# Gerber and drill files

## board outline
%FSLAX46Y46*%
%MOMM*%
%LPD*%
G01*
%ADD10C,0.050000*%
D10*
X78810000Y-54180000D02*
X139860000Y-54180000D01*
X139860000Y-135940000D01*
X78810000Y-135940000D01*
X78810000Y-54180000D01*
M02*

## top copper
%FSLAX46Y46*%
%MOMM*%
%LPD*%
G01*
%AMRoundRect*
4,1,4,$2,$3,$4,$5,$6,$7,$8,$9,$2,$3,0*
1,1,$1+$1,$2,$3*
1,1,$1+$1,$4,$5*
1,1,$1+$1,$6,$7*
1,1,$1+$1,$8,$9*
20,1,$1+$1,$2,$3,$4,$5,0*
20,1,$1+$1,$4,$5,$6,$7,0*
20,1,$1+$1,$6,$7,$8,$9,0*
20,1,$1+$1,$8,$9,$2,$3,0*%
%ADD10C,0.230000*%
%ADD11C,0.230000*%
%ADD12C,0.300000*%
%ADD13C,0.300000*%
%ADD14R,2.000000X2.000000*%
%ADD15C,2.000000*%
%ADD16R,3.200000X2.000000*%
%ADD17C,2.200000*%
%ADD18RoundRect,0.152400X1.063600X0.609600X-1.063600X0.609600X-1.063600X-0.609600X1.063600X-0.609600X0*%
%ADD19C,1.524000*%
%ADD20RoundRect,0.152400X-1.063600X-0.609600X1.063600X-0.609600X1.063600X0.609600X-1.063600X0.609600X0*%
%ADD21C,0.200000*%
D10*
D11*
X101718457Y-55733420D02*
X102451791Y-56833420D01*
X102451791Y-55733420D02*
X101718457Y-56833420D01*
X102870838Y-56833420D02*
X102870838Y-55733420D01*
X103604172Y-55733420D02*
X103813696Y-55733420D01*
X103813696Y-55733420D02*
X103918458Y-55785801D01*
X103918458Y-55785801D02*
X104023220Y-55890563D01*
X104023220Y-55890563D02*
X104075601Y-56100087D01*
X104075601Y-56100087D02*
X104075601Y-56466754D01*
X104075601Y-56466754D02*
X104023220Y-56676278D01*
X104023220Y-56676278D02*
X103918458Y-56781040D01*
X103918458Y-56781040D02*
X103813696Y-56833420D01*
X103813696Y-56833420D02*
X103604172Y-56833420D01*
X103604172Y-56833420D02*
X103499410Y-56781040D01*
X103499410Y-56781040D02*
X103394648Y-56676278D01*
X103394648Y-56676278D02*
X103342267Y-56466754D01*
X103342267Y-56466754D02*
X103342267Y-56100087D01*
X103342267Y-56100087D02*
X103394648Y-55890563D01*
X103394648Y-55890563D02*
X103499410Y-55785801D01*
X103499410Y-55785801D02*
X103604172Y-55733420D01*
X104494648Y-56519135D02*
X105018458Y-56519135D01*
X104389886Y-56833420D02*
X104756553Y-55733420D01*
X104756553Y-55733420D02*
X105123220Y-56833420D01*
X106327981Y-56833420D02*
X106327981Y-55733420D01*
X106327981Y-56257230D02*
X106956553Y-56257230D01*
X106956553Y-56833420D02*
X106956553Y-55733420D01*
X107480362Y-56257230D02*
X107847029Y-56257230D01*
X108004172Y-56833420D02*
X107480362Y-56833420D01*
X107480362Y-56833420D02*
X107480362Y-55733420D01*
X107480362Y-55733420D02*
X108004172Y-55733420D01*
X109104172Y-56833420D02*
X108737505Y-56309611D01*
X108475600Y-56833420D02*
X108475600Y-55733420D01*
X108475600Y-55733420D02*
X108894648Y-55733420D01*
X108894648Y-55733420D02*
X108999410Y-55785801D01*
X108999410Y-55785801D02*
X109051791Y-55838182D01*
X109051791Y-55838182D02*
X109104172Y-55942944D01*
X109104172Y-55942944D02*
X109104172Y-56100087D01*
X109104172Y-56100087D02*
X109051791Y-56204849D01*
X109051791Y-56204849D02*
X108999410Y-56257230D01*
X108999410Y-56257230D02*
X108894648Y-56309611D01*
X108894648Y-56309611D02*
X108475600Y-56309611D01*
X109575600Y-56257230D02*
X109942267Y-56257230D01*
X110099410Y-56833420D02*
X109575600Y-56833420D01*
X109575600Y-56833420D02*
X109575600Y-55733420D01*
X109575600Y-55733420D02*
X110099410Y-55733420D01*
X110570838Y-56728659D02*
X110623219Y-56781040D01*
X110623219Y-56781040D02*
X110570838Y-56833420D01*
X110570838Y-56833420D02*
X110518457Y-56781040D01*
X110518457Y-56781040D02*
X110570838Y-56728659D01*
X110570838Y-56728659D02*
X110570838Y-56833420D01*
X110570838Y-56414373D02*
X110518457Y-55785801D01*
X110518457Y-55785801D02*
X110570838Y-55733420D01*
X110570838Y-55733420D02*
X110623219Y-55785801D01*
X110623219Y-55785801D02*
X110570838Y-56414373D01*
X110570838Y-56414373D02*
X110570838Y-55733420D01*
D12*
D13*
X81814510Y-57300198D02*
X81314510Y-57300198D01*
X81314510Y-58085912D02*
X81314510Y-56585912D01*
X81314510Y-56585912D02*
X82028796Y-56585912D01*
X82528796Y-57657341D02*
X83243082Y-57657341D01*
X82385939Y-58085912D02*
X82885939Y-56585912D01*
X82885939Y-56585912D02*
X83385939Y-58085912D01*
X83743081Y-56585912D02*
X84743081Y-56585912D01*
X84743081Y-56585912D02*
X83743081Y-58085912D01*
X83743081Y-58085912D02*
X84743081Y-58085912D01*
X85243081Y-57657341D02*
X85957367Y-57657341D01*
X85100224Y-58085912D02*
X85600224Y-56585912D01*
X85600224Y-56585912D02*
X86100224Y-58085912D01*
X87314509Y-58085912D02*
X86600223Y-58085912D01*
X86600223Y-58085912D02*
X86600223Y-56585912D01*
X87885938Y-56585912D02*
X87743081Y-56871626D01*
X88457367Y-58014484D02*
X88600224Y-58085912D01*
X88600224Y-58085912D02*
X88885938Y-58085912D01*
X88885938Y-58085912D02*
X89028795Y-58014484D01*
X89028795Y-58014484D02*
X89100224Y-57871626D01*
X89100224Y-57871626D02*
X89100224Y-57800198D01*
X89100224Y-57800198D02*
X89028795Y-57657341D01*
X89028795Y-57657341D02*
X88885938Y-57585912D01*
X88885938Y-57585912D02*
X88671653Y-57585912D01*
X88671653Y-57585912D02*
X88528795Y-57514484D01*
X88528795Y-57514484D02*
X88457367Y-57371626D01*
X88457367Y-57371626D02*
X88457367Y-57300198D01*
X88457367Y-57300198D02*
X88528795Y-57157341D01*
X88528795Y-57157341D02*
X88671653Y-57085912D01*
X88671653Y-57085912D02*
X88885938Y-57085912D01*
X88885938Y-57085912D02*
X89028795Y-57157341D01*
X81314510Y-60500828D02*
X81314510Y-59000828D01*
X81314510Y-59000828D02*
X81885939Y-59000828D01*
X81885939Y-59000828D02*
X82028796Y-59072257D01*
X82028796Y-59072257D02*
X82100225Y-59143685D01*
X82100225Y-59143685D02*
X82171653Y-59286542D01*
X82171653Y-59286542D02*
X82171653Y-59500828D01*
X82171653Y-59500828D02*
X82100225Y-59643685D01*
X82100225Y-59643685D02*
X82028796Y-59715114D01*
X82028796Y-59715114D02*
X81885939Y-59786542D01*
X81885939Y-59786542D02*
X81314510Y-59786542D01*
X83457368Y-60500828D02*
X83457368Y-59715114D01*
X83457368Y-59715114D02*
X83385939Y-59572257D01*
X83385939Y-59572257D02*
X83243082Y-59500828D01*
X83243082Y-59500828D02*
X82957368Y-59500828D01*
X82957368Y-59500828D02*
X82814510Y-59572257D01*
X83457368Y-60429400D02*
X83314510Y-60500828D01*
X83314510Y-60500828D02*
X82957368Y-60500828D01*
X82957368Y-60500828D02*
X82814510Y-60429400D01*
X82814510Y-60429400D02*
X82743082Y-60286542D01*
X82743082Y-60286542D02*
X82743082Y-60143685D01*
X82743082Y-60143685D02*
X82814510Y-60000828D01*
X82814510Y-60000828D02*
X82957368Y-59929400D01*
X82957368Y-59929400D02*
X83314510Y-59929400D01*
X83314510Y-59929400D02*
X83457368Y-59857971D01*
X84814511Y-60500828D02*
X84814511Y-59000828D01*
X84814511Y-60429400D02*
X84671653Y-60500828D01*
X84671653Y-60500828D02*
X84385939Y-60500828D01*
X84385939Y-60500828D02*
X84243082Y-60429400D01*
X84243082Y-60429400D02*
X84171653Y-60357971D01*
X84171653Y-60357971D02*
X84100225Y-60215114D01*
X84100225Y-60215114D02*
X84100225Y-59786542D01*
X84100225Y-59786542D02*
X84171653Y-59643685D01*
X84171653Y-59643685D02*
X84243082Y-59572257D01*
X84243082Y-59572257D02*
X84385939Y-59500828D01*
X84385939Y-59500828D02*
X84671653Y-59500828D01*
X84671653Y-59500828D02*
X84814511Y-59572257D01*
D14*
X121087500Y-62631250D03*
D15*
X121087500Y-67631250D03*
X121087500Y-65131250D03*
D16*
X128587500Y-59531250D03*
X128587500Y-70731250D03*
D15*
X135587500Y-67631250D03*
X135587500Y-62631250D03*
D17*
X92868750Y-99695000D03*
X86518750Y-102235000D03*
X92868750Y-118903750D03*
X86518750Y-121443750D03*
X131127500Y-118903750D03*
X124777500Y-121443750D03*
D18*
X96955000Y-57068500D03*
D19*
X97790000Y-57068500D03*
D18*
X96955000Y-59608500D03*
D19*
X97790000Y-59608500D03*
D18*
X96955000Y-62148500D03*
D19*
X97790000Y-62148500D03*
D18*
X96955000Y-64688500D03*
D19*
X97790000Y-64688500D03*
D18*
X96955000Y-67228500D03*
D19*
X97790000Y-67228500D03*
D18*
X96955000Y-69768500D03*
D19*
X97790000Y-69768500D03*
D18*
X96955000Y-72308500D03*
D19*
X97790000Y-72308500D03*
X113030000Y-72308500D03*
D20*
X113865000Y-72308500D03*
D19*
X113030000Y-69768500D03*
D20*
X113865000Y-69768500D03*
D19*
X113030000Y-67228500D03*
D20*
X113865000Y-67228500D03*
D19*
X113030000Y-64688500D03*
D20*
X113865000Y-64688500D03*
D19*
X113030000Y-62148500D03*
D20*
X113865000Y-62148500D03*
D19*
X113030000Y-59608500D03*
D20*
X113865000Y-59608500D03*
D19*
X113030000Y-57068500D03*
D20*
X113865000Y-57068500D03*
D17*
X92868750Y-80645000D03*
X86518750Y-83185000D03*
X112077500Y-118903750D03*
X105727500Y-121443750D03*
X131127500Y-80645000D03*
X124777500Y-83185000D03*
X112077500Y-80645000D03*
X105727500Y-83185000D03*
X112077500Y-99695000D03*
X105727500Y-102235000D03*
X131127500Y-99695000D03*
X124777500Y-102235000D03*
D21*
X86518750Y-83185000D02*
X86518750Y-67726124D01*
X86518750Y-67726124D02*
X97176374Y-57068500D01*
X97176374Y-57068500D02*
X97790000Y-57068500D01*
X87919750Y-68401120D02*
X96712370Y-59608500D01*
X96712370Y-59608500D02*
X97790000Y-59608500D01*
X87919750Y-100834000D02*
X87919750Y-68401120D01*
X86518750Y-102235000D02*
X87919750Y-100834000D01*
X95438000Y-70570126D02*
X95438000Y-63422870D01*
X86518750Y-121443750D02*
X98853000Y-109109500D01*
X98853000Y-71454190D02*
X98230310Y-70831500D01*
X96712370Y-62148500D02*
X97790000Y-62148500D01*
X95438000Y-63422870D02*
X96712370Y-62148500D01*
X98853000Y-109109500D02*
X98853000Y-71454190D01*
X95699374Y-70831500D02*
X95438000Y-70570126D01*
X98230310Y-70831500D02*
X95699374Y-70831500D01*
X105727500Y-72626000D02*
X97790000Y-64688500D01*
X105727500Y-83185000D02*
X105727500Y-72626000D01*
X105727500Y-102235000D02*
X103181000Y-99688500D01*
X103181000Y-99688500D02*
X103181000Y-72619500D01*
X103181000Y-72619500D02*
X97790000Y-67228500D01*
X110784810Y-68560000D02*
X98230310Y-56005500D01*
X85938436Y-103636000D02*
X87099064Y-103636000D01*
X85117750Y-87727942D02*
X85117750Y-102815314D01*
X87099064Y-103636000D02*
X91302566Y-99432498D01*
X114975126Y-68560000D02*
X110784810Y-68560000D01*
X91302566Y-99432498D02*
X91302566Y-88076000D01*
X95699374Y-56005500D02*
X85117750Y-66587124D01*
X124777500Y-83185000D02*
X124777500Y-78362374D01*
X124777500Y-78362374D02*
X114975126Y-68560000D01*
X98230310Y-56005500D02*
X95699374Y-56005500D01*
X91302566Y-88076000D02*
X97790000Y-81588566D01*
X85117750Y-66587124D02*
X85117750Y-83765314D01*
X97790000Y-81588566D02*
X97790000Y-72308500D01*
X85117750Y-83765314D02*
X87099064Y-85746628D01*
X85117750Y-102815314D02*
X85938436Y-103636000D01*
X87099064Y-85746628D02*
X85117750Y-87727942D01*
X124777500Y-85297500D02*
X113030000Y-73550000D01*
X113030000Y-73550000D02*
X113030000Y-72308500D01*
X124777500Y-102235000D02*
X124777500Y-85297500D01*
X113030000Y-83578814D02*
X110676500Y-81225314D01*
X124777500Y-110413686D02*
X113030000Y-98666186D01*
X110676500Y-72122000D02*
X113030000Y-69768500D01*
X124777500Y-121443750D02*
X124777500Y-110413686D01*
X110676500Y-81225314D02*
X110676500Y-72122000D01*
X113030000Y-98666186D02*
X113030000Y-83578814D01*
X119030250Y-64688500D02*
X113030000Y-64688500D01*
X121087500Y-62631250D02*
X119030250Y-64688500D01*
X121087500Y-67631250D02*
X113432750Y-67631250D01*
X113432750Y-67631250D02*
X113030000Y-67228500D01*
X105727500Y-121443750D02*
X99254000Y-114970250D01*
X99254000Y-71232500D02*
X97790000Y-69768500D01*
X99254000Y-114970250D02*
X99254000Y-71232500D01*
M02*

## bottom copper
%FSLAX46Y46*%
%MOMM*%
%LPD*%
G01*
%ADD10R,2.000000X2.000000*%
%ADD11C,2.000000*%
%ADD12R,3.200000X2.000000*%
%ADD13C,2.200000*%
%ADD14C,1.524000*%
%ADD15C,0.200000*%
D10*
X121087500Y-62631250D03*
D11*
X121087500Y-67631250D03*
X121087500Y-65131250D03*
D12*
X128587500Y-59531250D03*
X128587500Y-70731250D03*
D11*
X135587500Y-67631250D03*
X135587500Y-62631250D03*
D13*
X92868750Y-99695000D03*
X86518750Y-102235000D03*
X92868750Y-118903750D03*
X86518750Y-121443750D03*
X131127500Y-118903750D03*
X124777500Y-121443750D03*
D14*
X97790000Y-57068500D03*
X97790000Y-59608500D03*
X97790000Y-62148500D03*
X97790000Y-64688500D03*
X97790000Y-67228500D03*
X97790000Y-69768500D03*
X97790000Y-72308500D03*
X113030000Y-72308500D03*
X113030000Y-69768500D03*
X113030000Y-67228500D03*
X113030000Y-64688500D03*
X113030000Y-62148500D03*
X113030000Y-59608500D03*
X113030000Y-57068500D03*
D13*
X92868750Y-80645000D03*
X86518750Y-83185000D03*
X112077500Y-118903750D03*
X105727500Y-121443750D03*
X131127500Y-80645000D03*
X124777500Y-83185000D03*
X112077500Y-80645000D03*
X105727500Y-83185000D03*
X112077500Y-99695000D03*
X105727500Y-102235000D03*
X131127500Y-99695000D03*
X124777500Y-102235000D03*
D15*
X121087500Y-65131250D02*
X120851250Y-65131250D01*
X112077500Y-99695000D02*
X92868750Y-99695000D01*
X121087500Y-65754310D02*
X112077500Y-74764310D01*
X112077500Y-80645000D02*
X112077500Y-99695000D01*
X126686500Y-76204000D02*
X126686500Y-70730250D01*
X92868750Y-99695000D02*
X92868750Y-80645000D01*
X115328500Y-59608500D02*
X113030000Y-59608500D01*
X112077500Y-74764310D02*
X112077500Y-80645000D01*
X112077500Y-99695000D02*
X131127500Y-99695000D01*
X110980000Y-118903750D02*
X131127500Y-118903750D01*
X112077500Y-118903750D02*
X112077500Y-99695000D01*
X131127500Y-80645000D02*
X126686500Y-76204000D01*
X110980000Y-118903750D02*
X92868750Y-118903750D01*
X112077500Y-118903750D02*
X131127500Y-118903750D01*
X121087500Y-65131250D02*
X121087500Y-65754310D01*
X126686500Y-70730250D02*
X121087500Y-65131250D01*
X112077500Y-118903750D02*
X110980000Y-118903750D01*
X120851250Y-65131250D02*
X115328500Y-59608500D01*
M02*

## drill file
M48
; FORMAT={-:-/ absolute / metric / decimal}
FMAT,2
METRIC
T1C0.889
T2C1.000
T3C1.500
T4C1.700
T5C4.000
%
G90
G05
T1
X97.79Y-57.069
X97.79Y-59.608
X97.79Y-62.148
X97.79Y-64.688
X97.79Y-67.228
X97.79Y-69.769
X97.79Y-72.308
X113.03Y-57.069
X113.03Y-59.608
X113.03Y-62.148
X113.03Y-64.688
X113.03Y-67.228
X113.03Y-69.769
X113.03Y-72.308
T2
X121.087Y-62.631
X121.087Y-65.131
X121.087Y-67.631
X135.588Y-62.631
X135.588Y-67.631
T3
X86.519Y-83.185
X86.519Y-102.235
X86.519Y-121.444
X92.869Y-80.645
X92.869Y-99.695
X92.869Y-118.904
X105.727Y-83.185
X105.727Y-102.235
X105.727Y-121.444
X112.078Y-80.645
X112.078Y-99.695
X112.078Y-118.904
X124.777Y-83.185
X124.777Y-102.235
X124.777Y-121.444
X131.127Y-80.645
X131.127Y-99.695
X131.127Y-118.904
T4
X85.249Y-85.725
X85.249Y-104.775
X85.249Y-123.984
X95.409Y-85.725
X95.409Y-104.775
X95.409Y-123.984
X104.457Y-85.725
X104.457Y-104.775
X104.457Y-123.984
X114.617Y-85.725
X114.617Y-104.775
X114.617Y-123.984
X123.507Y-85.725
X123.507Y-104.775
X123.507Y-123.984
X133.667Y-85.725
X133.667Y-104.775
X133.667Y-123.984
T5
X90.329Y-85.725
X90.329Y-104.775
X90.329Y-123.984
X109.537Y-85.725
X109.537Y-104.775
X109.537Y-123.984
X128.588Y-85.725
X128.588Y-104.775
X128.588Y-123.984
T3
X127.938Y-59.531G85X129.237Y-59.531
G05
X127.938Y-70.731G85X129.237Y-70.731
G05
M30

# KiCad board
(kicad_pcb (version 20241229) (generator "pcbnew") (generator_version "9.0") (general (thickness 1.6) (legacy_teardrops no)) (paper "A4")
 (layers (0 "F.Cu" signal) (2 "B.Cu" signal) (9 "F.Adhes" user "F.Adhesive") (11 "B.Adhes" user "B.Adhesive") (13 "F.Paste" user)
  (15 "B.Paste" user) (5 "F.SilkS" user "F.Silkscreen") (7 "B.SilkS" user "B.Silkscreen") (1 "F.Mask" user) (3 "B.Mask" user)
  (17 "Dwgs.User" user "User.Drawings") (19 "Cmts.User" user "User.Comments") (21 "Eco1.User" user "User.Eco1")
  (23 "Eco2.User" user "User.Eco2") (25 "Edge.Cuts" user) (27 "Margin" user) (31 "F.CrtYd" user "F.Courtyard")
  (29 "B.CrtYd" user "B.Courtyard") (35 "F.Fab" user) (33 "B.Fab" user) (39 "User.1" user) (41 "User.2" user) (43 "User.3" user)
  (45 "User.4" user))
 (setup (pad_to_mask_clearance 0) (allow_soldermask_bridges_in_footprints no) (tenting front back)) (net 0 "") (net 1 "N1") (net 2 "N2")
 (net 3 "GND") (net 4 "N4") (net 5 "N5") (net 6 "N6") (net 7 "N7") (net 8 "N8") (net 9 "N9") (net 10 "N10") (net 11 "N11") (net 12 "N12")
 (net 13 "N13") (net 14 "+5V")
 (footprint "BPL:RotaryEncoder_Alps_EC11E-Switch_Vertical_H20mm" (layer "F.Cu") (at 121.0875 62.63125)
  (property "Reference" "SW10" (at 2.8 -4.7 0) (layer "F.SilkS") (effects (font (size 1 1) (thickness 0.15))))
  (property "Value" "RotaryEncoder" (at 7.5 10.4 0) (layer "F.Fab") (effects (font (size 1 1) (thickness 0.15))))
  (pad "A" thru_hole rect (at 0 0) (size 2 2) (drill 1) (layers "*.Cu" "*.Mask") (remove_unused_layers no) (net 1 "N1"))
  (pad "B" thru_hole circle (at 0 5) (size 2 2) (drill 1) (layers "*.Cu" "*.Mask") (remove_unused_layers no) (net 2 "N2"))
  (pad "C" thru_hole circle (at 0 2.5) (size 2 2) (drill 1) (layers "*.Cu" "*.Mask") (remove_unused_layers no) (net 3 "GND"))
  (pad "MP" thru_hole rect (at 7.5 -3.1) (size 3.2 2) (drill oval 2.8 1.5) (layers "*.Cu" "*.Mask") (remove_unused_layers no))
  (pad "MP" thru_hole rect (at 7.5 8.1) (size 3.2 2) (drill oval 2.8 1.5) (layers "*.Cu" "*.Mask") (remove_unused_layers no))
  (pad "S1" thru_hole circle (at 14.5 5) (size 2 2) (drill 1) (layers "*.Cu" "*.Mask") (remove_unused_layers no))
  (pad "S2" thru_hole circle (at 14.5 0) (size 2 2) (drill 1) (layers "*.Cu" "*.Mask") (remove_unused_layers no)))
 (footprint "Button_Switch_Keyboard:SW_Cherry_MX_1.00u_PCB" (layer "F.Cu") (at 92.86875 99.695)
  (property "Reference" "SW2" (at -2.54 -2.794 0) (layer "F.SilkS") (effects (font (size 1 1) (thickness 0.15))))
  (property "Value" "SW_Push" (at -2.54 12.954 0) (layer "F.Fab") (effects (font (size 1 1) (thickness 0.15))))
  (pad "" np_thru_hole circle (at -7.62 5.08) (size 1.7 1.7) (drill 1.7) (layers "*.Cu" "*.Mask"))
  (pad "" np_thru_hole circle (at -2.54 5.08) (size 4 4) (drill 4) (layers "*.Cu" "*.Mask"))
  (pad "" np_thru_hole circle (at 2.54 5.08) (size 1.7 1.7) (drill 1.7) (layers "*.Cu" "*.Mask"))
  (pad "1" thru_hole circle (at 0 0) (size 2.2 2.2) (drill 1.5) (layers "*.Cu" "*.Mask") (remove_unused_layers no) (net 3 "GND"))
  (pad "2" thru_hole circle (at -6.35 2.54) (size 2.2 2.2) (drill 1.5) (layers "*.Cu" "*.Mask") (remove_unused_layers no) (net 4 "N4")))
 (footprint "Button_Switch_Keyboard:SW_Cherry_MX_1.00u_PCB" (layer "F.Cu") (at 92.86875 118.90375)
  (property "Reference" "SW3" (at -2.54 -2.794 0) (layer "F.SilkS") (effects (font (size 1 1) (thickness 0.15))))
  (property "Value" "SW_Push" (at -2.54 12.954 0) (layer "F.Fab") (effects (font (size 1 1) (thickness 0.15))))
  (pad "" np_thru_hole circle (at -7.62 5.08) (size 1.7 1.7) (drill 1.7) (layers "*.Cu" "*.Mask"))
  (pad "" np_thru_hole circle (at -2.54 5.08) (size 4 4) (drill 4) (layers "*.Cu" "*.Mask"))
  (pad "" np_thru_hole circle (at 2.54 5.08) (size 1.7 1.7) (drill 1.7) (layers "*.Cu" "*.Mask"))
  (pad "1" thru_hole circle (at 0 0) (size 2.2 2.2) (drill 1.5) (layers "*.Cu" "*.Mask") (remove_unused_layers no) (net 3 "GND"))
  (pad "2" thru_hole circle (at -6.35 2.54) (size 2.2 2.2) (drill 1.5) (layers "*.Cu" "*.Mask") (remove_unused_layers no) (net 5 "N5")))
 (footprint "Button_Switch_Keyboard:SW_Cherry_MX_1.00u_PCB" (layer "F.Cu") (at 131.1275 118.90375)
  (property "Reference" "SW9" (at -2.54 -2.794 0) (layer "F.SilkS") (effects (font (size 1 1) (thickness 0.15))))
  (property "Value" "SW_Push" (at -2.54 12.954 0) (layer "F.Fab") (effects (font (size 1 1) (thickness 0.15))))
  (pad "" np_thru_hole circle (at -7.62 5.08) (size 1.7 1.7) (drill 1.7) (layers "*.Cu" "*.Mask"))
  (pad "" np_thru_hole circle (at -2.54 5.08) (size 4 4) (drill 4) (layers "*.Cu" "*.Mask"))
  (pad "" np_thru_hole circle (at 2.54 5.08) (size 1.7 1.7) (drill 1.7) (layers "*.Cu" "*.Mask"))
  (pad "1" thru_hole circle (at 0 0) (size 2.2 2.2) (drill 1.5) (layers "*.Cu" "*.Mask") (remove_unused_layers no) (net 3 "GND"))
  (pad "2" thru_hole circle (at -6.35 2.54) (size 2.2 2.2) (drill 1.5) (layers "*.Cu" "*.Mask") (remove_unused_layers no) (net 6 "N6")))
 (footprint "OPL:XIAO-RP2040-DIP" (layer "F.Cu") (at 105.41 64.6885)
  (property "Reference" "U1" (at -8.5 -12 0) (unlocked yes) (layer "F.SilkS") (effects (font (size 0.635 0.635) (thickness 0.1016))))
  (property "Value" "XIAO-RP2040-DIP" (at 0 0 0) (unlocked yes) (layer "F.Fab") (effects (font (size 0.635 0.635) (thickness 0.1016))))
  (pad "1" smd roundrect (at -8.455 -7.62 180) (size 2.432 1.524) (layers "F.Cu" "F.Mask") (roundrect_rratio 0.1) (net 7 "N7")
   (thermal_bridge_angle 45))
  (pad "1" thru_hole circle (at -7.62 -7.62 180) (size 1.524 1.524) (drill 0.889) (layers "*.Cu" "*.Mask") (remove_unused_layers no)
   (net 7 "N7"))
  (pad "2" smd roundrect (at -8.455 -5.08 180) (size 2.432 1.524) (layers "F.Cu" "F.Mask") (roundrect_rratio 0.1) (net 4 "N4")
   (thermal_bridge_angle 45))
  (pad "2" thru_hole circle (at -7.62 -5.08 180) (size 1.524 1.524) (drill 0.889) (layers "*.Cu" "*.Mask") (remove_unused_layers no)
   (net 4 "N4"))
  (pad "3" smd roundrect (at -8.455 -2.54 180) (size 2.432 1.524) (layers "F.Cu" "F.Mask") (roundrect_rratio 0.1) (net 5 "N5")
   (thermal_bridge_angle 45))
  (pad "3" thru_hole circle (at -7.62 -2.54 180) (size 1.524 1.524) (drill 0.889) (layers "*.Cu" "*.Mask") (remove_unused_layers no)
   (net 5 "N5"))
  (pad "4" smd roundrect (at -8.455 0 180) (size 2.432 1.524) (layers "F.Cu" "F.Mask") (roundrect_rratio 0.1) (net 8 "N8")
   (thermal_bridge_angle 45))
  (pad "4" thru_hole circle (at -7.62 0 180) (size 1.524 1.524) (drill 0.889) (layers "*.Cu" "*.Mask") (remove_unused_layers no)
   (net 8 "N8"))
  (pad "5" smd roundrect (at -8.455 2.54 180) (size 2.432 1.524) (layers "F.Cu" "F.Mask") (roundrect_rratio 0.1) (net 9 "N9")
   (thermal_bridge_angle 45))
  (pad "5" thru_hole circle (at -7.62 2.54 180) (size 1.524 1.524) (drill 0.889) (layers "*.Cu" "*.Mask") (remove_unused_layers no)
   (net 9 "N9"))
  (pad "6" smd roundrect (at -8.455 5.08 180) (size 2.432 1.524) (layers "F.Cu" "F.Mask") (roundrect_rratio 0.1) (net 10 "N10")
   (thermal_bridge_angle 45))
  (pad "6" thru_hole circle (at -7.62 5.08 180) (size 1.524 1.524) (drill 0.889) (layers "*.Cu" "*.Mask") (remove_unused_layers no)
   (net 10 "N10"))
  (pad "7" smd roundrect (at -8.455 7.62 180) (size 2.432 1.524) (layers "F.Cu" "F.Mask") (roundrect_rratio 0.1) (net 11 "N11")
   (thermal_bridge_angle 45))
  (pad "7" thru_hole circle (at -7.62 7.62 180) (size 1.524 1.524) (drill 0.889) (layers "*.Cu" "*.Mask") (remove_unused_layers no)
   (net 11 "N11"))
  (pad "8" thru_hole circle (at 7.62 7.62) (size 1.524 1.524) (drill 0.889) (layers "*.Cu" "*.Mask") (remove_unused_layers no)
   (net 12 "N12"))
  (pad "8" smd roundrect (at 8.455 7.62) (size 2.432 1.524) (layers "F.Cu" "F.Mask") (roundrect_rratio 0.1) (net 12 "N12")
   (thermal_bridge_angle 45))
  (pad "9" thru_hole circle (at 7.62 5.08) (size 1.524 1.524) (drill 0.889) (layers "*.Cu" "*.Mask") (remove_unused_layers no) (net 6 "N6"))
  (pad "9" smd roundrect (at 8.455 5.08) (size 2.432 1.524) (layers "F.Cu" "F.Mask") (roundrect_rratio 0.1) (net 6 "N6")
   (thermal_bridge_angle 45))
  (pad "10" thru_hole circle (at 7.62 2.54) (size 1.524 1.524) (drill 0.889) (layers "*.Cu" "*.Mask") (remove_unused_layers no) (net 2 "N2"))
  (pad "10" smd roundrect (at 8.455 2.54) (size 2.432 1.524) (layers "F.Cu" "F.Mask") (roundrect_rratio 0.1) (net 2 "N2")
   (thermal_bridge_angle 45))
  (pad "11" thru_hole circle (at 7.62 0) (size 1.524 1.524) (drill 0.889) (layers "*.Cu" "*.Mask") (remove_unused_layers no) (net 1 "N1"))
  (pad "11" smd roundrect (at 8.455 0) (size 2.432 1.524) (layers "F.Cu" "F.Mask") (roundrect_rratio 0.1) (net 1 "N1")
   (thermal_bridge_angle 45))
  (pad "12" thru_hole circle (at 7.62 -2.54) (size 1.524 1.524) (drill 0.889) (layers "*.Cu" "*.Mask") (remove_unused_layers no)
   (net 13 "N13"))
  (pad "12" smd roundrect (at 8.455 -2.54) (size 2.432 1.524) (layers "F.Cu" "F.Mask") (roundrect_rratio 0.1) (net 13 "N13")
   (thermal_bridge_angle 45))
  (pad "13" thru_hole circle (at 7.62 -5.08) (size 1.524 1.524) (drill 0.889) (layers "*.Cu" "*.Mask") (remove_unused_layers no)
   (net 3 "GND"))
  (pad "13" smd roundrect (at 8.455 -5.08) (size 2.432 1.524) (layers "F.Cu" "F.Mask") (roundrect_rratio 0.1) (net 3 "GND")
   (thermal_bridge_angle 45))
  (pad "14" thru_hole circle (at 7.62 -7.62) (size 1.524 1.524) (drill 0.889) (layers "*.Cu" "*.Mask") (remove_unused_layers no)
   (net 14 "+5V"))
  (pad "14" smd roundrect (at 8.455 -7.62) (size 2.432 1.524) (layers "F.Cu" "F.Mask") (roundrect_rratio 0.1) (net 14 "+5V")
   (thermal_bridge_angle 45)))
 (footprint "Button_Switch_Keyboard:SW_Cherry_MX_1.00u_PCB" (layer "F.Cu") (at 92.86875 80.645)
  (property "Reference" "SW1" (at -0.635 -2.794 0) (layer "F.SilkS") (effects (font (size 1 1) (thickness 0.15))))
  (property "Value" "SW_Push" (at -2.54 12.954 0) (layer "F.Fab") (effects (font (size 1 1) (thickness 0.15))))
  (pad "" np_thru_hole circle (at -7.62 5.08) (size 1.7 1.7) (drill 1.7) (layers "*.Cu" "*.Mask"))
  (pad "" np_thru_hole circle (at -2.54 5.08) (size 4 4) (drill 4) (layers "*.Cu" "*.Mask"))
  (pad "" np_thru_hole circle (at 2.54 5.08) (size 1.7 1.7) (drill 1.7) (layers "*.Cu" "*.Mask"))
  (pad "1" thru_hole circle (at 0 0) (size 2.2 2.2) (drill 1.5) (layers "*.Cu" "*.Mask") (remove_unused_layers no) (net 3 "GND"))
  (pad "2" thru_hole circle (at -6.35 2.54) (size 2.2 2.2) (drill 1.5) (layers "*.Cu" "*.Mask") (remove_unused_layers no) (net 7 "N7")))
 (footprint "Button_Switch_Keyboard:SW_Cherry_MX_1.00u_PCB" (layer "F.Cu") (at 112.0775 118.90375)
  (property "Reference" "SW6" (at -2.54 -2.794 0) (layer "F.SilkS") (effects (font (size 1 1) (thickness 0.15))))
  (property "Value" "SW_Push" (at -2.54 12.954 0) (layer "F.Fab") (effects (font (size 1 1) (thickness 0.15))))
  (pad "" np_thru_hole circle (at -7.62 5.08) (size 1.7 1.7) (drill 1.7) (layers "*.Cu" "*.Mask"))
  (pad "" np_thru_hole circle (at -2.54 5.08) (size 4 4) (drill 4) (layers "*.Cu" "*.Mask"))
  (pad "" np_thru_hole circle (at 2.54 5.08) (size 1.7 1.7) (drill 1.7) (layers "*.Cu" "*.Mask"))
  (pad "1" thru_hole circle (at 0 0) (size 2.2 2.2) (drill 1.5) (layers "*.Cu" "*.Mask") (remove_unused_layers no) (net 3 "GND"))
  (pad "2" thru_hole circle (at -6.35 2.54) (size 2.2 2.2) (drill 1.5) (layers "*.Cu" "*.Mask") (remove_unused_layers no) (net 10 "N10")))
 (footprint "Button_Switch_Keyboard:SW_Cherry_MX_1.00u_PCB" (layer "F.Cu") (at 131.1275 80.645)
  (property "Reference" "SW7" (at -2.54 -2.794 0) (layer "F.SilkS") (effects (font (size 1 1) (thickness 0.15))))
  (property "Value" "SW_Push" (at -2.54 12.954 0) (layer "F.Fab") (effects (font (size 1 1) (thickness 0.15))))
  (pad "" np_thru_hole circle (at -7.62 5.08) (size 1.7 1.7) (drill 1.7) (layers "*.Cu" "*.Mask"))
  (pad "" np_thru_hole circle (at -2.54 5.08) (size 4 4) (drill 4) (layers "*.Cu" "*.Mask"))
  (pad "" np_thru_hole circle (at 2.54 5.08) (size 1.7 1.7) (drill 1.7) (layers "*.Cu" "*.Mask"))
  (pad "1" thru_hole circle (at 0 0) (size 2.2 2.2) (drill 1.5) (layers "*.Cu" "*.Mask") (remove_unused_layers no) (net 3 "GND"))
  (pad "2" thru_hole circle (at -6.35 2.54) (size 2.2 2.2) (drill 1.5) (layers "*.Cu" "*.Mask") (remove_unused_layers no) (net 11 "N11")))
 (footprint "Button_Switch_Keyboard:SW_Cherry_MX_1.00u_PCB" (layer "F.Cu") (at 112.0775 80.645)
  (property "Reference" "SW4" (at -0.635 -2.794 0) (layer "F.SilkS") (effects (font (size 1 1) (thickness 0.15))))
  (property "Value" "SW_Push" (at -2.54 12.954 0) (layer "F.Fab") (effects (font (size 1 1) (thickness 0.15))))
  (pad "" np_thru_hole circle (at -7.62 5.08) (size 1.7 1.7) (drill 1.7) (layers "*.Cu" "*.Mask"))
  (pad "" np_thru_hole circle (at -2.54 5.08) (size 4 4) (drill 4) (layers "*.Cu" "*.Mask"))
  (pad "" np_thru_hole circle (at 2.54 5.08) (size 1.7 1.7) (drill 1.7) (layers "*.Cu" "*.Mask"))
  (pad "1" thru_hole circle (at 0 0) (size 2.2 2.2) (drill 1.5) (layers "*.Cu" "*.Mask") (remove_unused_layers no) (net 3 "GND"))
  (pad "2" thru_hole circle (at -6.35 2.54) (size 2.2 2.2) (drill 1.5) (layers "*.Cu" "*.Mask") (remove_unused_layers no) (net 8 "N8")))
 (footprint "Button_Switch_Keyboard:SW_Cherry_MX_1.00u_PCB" (layer "F.Cu") (at 112.0775 99.695)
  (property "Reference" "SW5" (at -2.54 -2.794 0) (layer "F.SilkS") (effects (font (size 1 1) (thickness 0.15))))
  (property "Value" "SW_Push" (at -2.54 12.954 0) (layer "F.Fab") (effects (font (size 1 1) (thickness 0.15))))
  (pad "" np_thru_hole circle (at -7.62 5.08) (size 1.7 1.7) (drill 1.7) (layers "*.Cu" "*.Mask"))
  (pad "" np_thru_hole circle (at -2.54 5.08) (size 4 4) (drill 4) (layers "*.Cu" "*.Mask"))
  (pad "" np_thru_hole circle (at 2.54 5.08) (size 1.7 1.7) (drill 1.7) (layers "*.Cu" "*.Mask"))
  (pad "1" thru_hole circle (at 0 0) (size 2.2 2.2) (drill 1.5) (layers "*.Cu" "*.Mask") (remove_unused_layers no) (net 3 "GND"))
  (pad "2" thru_hole circle (at -6.35 2.54) (size 2.2 2.2) (drill 1.5) (layers "*.Cu" "*.Mask") (remove_unused_layers no) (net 9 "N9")))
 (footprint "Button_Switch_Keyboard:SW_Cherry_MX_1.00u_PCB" (layer "F.Cu") (at 131.1275 99.695)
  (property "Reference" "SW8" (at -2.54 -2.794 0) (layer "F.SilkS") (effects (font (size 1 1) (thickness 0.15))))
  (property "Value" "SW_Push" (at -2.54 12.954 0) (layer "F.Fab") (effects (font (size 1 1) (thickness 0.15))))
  (pad "" np_thru_hole circle (at -7.62 5.08) (size 1.7 1.7) (drill 1.7) (layers "*.Cu" "*.Mask"))
  (pad "" np_thru_hole circle (at -2.54 5.08) (size 4 4) (drill 4) (layers "*.Cu" "*.Mask"))
  (pad "" np_thru_hole circle (at 2.54 5.08) (size 1.7 1.7) (drill 1.7) (layers "*.Cu" "*.Mask"))
  (pad "1" thru_hole circle (at 0 0) (size 2.2 2.2) (drill 1.5) (layers "*.Cu" "*.Mask") (remove_unused_layers no) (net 3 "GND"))
  (pad "2" thru_hole circle (at -6.35 2.54) (size 2.2 2.2) (drill 1.5) (layers "*.Cu" "*.Mask") (remove_unused_layers no) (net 12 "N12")))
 (gr_rect (start 78.81 54.18) (end 139.86 135.94) (stroke (width 0.05) (type default)) (fill no) (layer "Edge.Cuts"))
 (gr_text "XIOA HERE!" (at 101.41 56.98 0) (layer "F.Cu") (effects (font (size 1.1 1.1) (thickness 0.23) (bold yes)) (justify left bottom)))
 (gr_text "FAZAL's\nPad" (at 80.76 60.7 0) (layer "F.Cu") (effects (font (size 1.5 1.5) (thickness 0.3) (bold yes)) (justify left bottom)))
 (segment (start 86.51875 83.185) (end 86.51875 67.726124) (width 0.2) (layer "F.Cu") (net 7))
 (segment (start 86.51875 67.726124) (end 97.176374 57.0685) (width 0.2) (layer "F.Cu") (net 7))
 (segment (start 97.176374 57.0685) (end 97.79 57.0685) (width 0.2) (layer "F.Cu") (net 7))
 (segment (start 121.0875 65.13125) (end 120.85125 65.13125) (width 0.2) (layer "B.Cu") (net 3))
 (segment (start 112.0775 99.695) (end 92.86875 99.695) (width 0.2) (layer "B.Cu") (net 3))
 (segment (start 121.0875 65.75431) (end 112.0775 74.76431) (width 0.2) (layer "B.Cu") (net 3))
 (segment (start 112.0775 80.645) (end 112.0775 99.695) (width 0.2) (layer "B.Cu") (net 3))
 (segment (start 126.6865 76.204) (end 126.6865 70.73025) (width 0.2) (layer "B.Cu") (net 3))
 (segment (start 92.86875 99.695) (end 92.86875 80.645) (width 0.2) (layer "B.Cu") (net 3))
 (segment (start 115.3285 59.6085) (end 113.03 59.6085) (width 0.2) (layer "B.Cu") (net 3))
 (segment (start 112.0775 74.76431) (end 112.0775 80.645) (width 0.2) (layer "B.Cu") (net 3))
 (segment (start 112.0775 99.695) (end 131.1275 99.695) (width 0.2) (layer "B.Cu") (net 3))
 (segment (start 110.98 118.90375) (end 131.1275 118.90375) (width 0.2) (layer "B.Cu") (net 3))
 (segment (start 112.0775 118.90375) (end 112.0775 99.695) (width 0.2) (layer "B.Cu") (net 3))
 (segment (start 131.1275 80.645) (end 126.6865 76.204) (width 0.2) (layer "B.Cu") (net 3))
 (segment (start 110.98 118.90375) (end 92.86875 118.90375) (width 0.2) (layer "B.Cu") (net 3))
 (segment (start 112.0775 118.90375) (end 131.1275 118.90375) (width 0.2) (layer "B.Cu") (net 3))
 (segment (start 121.0875 65.13125) (end 121.0875 65.75431) (width 0.2) (layer "B.Cu") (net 3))
 (segment (start 126.6865 70.73025) (end 121.0875 65.13125) (width 0.2) (layer "B.Cu") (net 3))
 (segment (start 112.0775 118.90375) (end 110.98 118.90375) (width 0.2) (layer "B.Cu") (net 3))
 (segment (start 120.85125 65.13125) (end 115.3285 59.6085) (width 0.2) (layer "B.Cu") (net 3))
 (segment (start 87.91975 68.40112) (end 96.71237 59.6085) (width 0.2) (layer "F.Cu") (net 4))
 (segment (start 96.71237 59.6085) (end 97.79 59.6085) (width 0.2) (layer "F.Cu") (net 4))
 (segment (start 87.91975 100.834) (end 87.91975 68.40112) (width 0.2) (layer "F.Cu") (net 4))
 (segment (start 86.51875 102.235) (end 87.91975 100.834) (width 0.2) (layer "F.Cu") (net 4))
 (segment (start 95.438 70.570126) (end 95.438 63.42287) (width 0.2) (layer "F.Cu") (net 5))
 (segment (start 86.51875 121.44375) (end 98.853 109.1095) (width 0.2) (layer "F.Cu") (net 5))
 (segment (start 98.853 71.45419) (end 98.23031 70.8315) (width 0.2) (layer "F.Cu") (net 5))
 (segment (start 96.71237 62.1485) (end 97.79 62.1485) (width 0.2) (layer "F.Cu") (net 5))
 (segment (start 95.438 63.42287) (end 96.71237 62.1485) (width 0.2) (layer "F.Cu") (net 5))
 (segment (start 98.853 109.1095) (end 98.853 71.45419) (width 0.2) (layer "F.Cu") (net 5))
 (segment (start 95.699374 70.8315) (end 95.438 70.570126) (width 0.2) (layer "F.Cu") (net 5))
 (segment (start 98.23031 70.8315) (end 95.699374 70.8315) (width 0.2) (layer "F.Cu") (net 5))
 (segment (start 105.7275 72.626) (end 97.79 64.6885) (width 0.2) (layer "F.Cu") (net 8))
 (segment (start 105.7275 83.185) (end 105.7275 72.626) (width 0.2) (layer "F.Cu") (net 8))
 (segment (start 105.7275 102.235) (end 103.181 99.6885) (width 0.2) (layer "F.Cu") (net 9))
 (segment (start 103.181 99.6885) (end 103.181 72.6195) (width 0.2) (layer "F.Cu") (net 9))
 (segment (start 103.181 72.6195) (end 97.79 67.2285) (width 0.2) (layer "F.Cu") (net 9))
 (segment (start 110.78481 68.56) (end 98.23031 56.0055) (width 0.2) (layer "F.Cu") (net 11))
 (segment (start 85.938436 103.636) (end 87.099064 103.636) (width 0.2) (layer "F.Cu") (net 11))
 (segment (start 85.11775 87.727942) (end 85.11775 102.815314) (width 0.2) (layer "F.Cu") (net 11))
 (segment (start 87.099064 103.636) (end 91.302566 99.432498) (width 0.2) (layer "F.Cu") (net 11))
 (segment (start 114.975126 68.56) (end 110.78481 68.56) (width 0.2) (layer "F.Cu") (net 11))
 (segment (start 91.302566 99.432498) (end 91.302566 88.076) (width 0.2) (layer "F.Cu") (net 11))
 (segment (start 95.699374 56.0055) (end 85.11775 66.587124) (width 0.2) (layer "F.Cu") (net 11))
 (segment (start 124.7775 83.185) (end 124.7775 78.362374) (width 0.2) (layer "F.Cu") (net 11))
 (segment (start 124.7775 78.362374) (end 114.975126 68.56) (width 0.2) (layer "F.Cu") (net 11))
 (segment (start 98.23031 56.0055) (end 95.699374 56.0055) (width 0.2) (layer "F.Cu") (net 11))
 (segment (start 91.302566 88.076) (end 97.79 81.588566) (width 0.2) (layer "F.Cu") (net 11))
 (segment (start 85.11775 66.587124) (end 85.11775 83.765314) (width 0.2) (layer "F.Cu") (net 11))
 (segment (start 97.79 81.588566) (end 97.79 72.3085) (width 0.2) (layer "F.Cu") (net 11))
 (segment (start 85.11775 83.765314) (end 87.099064 85.746628) (width 0.2) (layer "F.Cu") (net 11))
 (segment (start 85.11775 102.815314) (end 85.938436 103.636) (width 0.2) (layer "F.Cu") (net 11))
 (segment (start 87.099064 85.746628) (end 85.11775 87.727942) (width 0.2) (layer "F.Cu") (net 11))
 (segment (start 124.7775 85.2975) (end 113.03 73.55) (width 0.2) (layer "F.Cu") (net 12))
 (segment (start 113.03 73.55) (end 113.03 72.3085) (width 0.2) (layer "F.Cu") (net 12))
 (segment (start 124.7775 102.235) (end 124.7775 85.2975) (width 0.2) (layer "F.Cu") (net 12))
 (segment (start 113.03 83.578814) (end 110.6765 81.225314) (width 0.2) (layer "F.Cu") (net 6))
 (segment (start 124.7775 110.413686) (end 113.03 98.666186) (width 0.2) (layer "F.Cu") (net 6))
 (segment (start 110.6765 72.122) (end 113.03 69.7685) (width 0.2) (layer "F.Cu") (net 6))
 (segment (start 124.7775 121.44375) (end 124.7775 110.413686) (width 0.2) (layer "F.Cu") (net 6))
 (segment (start 110.6765 81.225314) (end 110.6765 72.122) (width 0.2) (layer "F.Cu") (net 6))
 (segment (start 113.03 98.666186) (end 113.03 83.578814) (width 0.2) (layer "F.Cu") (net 6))
 (segment (start 119.03025 64.6885) (end 113.03 64.6885) (width 0.2) (layer "F.Cu") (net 1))
 (segment (start 121.0875 62.63125) (end 119.03025 64.6885) (width 0.2) (layer "F.Cu") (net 1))
 (segment (start 121.0875 67.63125) (end 113.43275 67.63125) (width 0.2) (layer "F.Cu") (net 2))
 (segment (start 113.43275 67.63125) (end 113.03 67.2285) (width 0.2) (layer "F.Cu") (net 2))
 (segment (start 105.7275 121.44375) (end 99.254 114.97025) (width 0.2) (layer "F.Cu") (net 10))
 (segment (start 99.254 71.2325) (end 97.79 69.7685) (width 0.2) (layer "F.Cu") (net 10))
 (segment (start 99.254 114.97025) (end 99.254 71.2325) (width 0.2) (layer "F.Cu") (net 10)))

